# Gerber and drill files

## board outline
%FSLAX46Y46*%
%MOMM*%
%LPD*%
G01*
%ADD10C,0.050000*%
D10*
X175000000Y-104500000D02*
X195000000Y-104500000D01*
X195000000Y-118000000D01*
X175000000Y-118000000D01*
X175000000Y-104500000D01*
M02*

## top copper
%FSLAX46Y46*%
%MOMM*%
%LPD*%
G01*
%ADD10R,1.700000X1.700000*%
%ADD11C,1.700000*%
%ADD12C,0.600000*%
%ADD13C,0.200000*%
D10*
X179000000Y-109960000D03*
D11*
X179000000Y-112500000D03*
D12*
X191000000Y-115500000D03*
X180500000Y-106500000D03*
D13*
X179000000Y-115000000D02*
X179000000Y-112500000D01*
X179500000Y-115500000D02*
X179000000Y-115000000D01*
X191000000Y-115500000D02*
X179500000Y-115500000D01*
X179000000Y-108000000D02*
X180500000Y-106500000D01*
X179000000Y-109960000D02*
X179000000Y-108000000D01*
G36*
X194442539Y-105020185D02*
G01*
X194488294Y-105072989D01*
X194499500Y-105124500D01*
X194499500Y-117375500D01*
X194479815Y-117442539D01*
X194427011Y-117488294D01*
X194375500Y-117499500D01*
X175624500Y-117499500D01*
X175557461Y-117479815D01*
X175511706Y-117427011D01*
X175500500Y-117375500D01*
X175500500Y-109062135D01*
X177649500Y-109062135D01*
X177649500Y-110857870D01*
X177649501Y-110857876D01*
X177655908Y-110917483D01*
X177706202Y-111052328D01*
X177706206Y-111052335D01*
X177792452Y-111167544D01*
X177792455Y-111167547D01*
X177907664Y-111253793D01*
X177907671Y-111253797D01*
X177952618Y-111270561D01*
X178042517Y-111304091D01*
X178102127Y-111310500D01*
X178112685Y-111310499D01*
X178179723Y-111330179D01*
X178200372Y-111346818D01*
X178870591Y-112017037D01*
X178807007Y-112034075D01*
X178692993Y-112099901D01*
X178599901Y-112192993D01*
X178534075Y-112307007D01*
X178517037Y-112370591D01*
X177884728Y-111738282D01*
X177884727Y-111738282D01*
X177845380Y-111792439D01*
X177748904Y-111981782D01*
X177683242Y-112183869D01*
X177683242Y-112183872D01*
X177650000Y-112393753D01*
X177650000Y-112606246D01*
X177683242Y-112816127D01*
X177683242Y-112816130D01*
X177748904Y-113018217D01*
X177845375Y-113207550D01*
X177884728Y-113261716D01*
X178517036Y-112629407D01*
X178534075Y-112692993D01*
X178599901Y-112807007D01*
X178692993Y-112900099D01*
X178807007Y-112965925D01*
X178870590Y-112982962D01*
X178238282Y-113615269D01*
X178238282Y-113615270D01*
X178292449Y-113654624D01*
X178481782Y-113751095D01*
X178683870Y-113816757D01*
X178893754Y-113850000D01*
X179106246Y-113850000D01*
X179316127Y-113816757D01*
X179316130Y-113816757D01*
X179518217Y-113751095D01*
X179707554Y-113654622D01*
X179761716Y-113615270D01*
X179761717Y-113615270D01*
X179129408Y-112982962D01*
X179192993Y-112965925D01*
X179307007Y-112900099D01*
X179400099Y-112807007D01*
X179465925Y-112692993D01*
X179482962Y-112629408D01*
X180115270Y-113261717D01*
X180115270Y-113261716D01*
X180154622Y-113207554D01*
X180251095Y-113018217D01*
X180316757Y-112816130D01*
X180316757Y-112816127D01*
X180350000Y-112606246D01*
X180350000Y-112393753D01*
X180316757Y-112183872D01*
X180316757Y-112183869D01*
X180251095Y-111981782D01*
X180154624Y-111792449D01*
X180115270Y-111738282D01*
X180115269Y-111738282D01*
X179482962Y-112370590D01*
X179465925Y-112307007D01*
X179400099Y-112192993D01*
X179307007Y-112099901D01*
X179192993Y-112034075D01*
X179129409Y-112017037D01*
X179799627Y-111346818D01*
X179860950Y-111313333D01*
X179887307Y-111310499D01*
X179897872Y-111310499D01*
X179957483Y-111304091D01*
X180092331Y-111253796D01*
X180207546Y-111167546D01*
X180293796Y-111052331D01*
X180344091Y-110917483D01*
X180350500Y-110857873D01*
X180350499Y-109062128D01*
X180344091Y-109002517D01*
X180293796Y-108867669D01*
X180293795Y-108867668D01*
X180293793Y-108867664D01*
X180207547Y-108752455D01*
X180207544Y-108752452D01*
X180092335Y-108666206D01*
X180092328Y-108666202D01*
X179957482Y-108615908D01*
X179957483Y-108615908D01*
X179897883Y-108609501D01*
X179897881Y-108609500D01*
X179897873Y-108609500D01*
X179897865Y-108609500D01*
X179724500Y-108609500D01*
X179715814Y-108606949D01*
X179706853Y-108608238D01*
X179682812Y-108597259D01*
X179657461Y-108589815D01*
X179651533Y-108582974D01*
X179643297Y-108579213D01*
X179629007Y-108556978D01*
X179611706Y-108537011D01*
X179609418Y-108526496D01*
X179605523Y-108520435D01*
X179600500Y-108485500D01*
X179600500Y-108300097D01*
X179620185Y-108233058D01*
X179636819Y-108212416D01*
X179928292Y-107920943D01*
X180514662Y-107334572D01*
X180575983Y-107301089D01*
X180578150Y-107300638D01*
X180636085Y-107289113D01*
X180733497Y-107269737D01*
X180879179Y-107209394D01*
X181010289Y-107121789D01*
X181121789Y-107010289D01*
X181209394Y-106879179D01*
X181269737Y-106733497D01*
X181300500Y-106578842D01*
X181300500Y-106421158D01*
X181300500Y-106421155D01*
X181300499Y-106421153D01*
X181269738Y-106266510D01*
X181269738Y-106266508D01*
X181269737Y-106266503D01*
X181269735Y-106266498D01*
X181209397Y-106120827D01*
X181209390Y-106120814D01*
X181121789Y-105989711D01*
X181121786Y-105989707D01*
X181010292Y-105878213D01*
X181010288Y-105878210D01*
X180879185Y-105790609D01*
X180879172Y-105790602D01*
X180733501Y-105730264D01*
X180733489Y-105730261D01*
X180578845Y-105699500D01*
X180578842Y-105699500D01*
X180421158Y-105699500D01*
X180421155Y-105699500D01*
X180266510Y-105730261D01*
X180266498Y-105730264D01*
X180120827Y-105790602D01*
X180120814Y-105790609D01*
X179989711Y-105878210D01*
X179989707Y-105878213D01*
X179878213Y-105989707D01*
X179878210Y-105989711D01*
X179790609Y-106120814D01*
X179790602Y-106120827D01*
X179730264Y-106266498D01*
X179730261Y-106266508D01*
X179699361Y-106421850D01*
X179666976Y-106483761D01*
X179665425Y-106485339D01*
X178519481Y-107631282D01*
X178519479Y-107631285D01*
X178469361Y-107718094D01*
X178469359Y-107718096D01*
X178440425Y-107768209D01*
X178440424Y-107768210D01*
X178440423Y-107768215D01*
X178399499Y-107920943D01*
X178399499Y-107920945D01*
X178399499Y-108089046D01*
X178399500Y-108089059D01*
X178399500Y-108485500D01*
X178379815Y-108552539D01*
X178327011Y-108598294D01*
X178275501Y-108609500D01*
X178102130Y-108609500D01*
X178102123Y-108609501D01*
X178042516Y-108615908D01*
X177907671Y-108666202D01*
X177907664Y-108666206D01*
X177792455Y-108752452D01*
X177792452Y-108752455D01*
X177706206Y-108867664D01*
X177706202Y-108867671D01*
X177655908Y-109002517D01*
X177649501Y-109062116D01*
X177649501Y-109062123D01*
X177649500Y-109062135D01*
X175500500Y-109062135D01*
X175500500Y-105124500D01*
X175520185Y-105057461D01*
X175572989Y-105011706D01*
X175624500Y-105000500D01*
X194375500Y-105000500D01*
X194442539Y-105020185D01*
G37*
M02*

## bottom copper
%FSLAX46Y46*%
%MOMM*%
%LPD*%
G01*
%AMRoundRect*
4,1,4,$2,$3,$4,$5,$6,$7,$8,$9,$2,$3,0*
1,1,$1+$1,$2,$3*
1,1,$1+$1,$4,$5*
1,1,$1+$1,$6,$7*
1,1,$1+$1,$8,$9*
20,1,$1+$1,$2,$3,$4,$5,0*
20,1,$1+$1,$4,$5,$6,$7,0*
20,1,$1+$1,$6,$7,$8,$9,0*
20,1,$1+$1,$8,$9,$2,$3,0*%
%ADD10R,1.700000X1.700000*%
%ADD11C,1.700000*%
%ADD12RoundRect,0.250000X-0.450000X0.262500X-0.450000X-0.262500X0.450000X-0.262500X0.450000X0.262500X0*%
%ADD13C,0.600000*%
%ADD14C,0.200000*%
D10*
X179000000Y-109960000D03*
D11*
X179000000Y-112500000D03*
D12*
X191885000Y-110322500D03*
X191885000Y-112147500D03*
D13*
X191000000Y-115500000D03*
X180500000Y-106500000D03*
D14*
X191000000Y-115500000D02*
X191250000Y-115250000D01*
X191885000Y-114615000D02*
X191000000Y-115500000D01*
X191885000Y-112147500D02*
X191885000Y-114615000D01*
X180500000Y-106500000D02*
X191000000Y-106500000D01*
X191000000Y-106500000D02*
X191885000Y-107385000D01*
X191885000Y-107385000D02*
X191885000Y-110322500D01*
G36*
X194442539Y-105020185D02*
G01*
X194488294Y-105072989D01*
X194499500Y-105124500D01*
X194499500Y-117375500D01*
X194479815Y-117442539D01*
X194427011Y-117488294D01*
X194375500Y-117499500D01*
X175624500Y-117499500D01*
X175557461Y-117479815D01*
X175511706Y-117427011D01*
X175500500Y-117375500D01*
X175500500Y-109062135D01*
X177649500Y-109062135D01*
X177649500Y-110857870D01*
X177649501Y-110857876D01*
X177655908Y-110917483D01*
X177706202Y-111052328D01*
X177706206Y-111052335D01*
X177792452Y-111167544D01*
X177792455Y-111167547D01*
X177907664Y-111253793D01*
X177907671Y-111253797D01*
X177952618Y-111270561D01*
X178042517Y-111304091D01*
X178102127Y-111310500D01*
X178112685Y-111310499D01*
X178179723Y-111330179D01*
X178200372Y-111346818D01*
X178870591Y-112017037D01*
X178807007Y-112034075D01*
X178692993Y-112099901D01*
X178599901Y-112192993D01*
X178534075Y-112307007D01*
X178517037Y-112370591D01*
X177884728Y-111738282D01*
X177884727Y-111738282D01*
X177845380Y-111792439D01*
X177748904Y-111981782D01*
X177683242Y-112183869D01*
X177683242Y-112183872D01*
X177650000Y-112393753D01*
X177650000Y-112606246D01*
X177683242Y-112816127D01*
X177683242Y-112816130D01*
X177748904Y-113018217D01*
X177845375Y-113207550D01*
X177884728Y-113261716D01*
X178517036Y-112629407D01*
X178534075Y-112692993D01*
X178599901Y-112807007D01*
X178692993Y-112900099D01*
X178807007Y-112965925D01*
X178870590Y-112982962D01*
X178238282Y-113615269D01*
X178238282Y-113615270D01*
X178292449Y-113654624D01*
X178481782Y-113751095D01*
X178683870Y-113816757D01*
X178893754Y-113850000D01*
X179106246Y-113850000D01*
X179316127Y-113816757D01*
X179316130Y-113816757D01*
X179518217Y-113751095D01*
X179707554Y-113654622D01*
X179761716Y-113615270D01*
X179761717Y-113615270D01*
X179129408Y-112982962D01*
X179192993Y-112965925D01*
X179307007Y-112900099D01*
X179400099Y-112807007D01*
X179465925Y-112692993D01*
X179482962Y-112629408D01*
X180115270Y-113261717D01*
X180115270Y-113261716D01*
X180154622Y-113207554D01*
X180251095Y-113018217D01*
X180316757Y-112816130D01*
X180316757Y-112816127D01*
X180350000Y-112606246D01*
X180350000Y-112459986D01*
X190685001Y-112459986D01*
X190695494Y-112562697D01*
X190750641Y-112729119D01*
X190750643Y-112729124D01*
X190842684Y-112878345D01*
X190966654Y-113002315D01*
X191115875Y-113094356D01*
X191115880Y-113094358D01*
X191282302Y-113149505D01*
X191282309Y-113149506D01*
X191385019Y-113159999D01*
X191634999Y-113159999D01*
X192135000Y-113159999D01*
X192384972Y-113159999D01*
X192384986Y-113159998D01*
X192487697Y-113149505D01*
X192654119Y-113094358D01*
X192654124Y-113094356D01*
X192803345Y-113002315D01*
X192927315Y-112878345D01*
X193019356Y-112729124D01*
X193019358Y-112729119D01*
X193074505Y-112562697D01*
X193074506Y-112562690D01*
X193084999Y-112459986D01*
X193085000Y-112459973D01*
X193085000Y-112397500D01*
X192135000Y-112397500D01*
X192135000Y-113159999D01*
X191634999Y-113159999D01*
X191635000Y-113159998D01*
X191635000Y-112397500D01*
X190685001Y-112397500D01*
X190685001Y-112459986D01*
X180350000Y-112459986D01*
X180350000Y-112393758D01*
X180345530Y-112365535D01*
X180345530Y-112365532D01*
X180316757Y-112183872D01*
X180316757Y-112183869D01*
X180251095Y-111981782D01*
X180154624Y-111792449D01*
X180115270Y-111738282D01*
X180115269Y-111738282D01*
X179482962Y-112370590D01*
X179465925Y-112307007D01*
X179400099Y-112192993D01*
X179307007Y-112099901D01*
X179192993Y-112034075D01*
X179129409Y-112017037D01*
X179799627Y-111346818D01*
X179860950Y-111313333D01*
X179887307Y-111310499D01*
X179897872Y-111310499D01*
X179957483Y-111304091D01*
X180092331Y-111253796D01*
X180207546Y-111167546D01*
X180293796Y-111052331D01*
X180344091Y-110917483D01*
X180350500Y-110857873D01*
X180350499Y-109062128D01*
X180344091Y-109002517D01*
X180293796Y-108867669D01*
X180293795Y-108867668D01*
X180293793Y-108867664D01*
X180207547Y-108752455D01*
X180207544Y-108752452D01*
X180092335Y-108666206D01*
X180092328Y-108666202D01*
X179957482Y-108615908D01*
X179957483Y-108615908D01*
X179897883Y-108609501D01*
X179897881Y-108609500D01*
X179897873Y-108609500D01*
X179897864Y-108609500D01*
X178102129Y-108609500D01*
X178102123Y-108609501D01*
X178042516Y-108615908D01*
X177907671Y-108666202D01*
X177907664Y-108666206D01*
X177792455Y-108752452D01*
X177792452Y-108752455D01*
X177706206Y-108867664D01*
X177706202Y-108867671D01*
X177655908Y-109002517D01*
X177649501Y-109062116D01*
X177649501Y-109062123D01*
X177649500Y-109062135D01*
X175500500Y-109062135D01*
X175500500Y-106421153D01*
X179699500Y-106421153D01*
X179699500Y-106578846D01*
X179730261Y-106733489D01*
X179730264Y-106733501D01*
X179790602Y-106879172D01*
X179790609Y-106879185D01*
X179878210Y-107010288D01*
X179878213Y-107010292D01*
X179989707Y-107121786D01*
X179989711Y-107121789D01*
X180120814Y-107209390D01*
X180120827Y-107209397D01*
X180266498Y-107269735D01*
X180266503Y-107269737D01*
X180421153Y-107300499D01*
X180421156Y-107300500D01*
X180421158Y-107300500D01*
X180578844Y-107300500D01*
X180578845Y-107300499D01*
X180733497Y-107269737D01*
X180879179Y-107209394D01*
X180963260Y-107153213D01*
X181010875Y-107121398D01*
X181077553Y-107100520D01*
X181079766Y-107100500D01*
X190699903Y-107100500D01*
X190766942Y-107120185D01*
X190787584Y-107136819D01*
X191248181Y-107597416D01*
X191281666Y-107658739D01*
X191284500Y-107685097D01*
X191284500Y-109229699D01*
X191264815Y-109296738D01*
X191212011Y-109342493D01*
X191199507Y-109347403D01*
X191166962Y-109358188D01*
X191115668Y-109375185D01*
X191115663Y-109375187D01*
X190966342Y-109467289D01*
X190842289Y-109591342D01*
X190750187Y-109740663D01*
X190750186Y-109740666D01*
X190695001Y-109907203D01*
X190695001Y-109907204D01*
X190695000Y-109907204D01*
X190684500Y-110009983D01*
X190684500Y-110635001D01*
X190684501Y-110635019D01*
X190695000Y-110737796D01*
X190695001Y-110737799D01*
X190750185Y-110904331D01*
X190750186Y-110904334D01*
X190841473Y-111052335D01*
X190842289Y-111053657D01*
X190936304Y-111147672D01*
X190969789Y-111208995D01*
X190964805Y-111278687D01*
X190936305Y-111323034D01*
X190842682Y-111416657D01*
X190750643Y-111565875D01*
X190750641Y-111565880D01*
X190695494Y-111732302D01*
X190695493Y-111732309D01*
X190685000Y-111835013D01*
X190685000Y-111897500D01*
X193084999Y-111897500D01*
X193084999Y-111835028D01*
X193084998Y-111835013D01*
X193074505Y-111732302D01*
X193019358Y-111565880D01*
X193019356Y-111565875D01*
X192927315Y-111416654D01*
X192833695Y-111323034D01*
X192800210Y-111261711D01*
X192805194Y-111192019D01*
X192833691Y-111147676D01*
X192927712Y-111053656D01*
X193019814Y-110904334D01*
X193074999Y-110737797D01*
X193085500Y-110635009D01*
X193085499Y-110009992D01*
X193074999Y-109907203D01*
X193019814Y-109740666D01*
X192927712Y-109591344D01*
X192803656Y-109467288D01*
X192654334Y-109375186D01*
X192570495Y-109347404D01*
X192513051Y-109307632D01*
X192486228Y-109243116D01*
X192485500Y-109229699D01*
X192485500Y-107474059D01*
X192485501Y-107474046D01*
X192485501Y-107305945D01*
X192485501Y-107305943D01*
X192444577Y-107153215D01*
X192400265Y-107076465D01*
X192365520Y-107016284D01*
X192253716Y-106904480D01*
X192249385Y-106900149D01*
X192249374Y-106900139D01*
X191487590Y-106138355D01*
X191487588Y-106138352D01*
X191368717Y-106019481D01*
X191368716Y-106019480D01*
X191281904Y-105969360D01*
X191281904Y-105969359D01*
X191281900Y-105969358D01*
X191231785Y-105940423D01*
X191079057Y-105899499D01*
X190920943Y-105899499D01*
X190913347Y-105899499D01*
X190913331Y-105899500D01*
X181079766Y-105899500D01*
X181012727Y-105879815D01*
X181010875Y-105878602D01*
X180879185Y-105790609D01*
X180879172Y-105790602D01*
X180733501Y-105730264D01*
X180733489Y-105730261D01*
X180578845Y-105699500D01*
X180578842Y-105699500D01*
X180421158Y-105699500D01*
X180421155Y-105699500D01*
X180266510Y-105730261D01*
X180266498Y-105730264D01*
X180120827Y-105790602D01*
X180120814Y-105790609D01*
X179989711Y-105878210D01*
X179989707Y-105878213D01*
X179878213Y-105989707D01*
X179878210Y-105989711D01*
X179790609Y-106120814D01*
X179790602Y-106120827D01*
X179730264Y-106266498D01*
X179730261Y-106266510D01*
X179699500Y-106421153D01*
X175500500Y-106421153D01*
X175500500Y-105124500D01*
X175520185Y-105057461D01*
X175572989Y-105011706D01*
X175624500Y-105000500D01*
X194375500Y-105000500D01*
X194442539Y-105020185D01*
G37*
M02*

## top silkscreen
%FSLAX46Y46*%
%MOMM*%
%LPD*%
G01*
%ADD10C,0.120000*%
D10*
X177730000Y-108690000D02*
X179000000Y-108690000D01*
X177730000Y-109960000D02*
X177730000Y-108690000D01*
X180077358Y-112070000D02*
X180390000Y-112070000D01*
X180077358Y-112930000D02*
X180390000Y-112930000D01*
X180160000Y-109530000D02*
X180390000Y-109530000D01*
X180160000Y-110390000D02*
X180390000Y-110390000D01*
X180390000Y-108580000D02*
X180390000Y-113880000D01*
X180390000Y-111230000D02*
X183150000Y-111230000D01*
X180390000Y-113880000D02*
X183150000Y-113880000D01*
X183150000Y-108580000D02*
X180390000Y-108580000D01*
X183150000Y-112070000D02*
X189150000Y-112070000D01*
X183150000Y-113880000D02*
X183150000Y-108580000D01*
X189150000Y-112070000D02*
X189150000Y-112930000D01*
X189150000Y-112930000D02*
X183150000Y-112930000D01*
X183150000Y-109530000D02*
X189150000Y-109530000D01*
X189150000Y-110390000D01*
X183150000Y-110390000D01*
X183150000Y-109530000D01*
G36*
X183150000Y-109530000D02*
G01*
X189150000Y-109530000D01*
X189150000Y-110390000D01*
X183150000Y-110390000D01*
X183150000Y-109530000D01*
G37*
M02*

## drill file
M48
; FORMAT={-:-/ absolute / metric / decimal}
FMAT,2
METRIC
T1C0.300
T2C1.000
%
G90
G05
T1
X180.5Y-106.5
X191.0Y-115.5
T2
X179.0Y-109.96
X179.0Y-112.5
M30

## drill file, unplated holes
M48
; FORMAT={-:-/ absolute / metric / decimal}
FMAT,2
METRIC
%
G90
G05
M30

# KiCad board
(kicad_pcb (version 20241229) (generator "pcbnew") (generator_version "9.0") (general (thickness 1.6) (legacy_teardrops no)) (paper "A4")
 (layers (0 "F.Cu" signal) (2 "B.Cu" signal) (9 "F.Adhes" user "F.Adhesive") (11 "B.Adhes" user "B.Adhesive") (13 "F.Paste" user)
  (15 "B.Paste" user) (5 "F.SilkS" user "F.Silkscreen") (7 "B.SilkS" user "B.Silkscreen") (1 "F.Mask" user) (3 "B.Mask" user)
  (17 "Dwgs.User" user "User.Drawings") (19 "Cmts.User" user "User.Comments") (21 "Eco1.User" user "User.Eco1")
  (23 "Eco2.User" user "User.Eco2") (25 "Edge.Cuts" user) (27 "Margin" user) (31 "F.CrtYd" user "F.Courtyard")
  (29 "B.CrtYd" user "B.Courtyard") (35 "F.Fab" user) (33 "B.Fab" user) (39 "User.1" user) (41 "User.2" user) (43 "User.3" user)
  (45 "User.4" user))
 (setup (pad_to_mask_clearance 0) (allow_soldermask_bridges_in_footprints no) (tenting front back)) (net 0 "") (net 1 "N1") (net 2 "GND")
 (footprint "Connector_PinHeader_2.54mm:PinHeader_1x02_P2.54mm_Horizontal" (layer "F.Cu") (at 179 109.96)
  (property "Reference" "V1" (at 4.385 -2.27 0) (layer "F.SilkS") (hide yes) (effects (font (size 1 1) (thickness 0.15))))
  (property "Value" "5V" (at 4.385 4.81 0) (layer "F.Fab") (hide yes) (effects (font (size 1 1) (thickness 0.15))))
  (fp_line (start -1.27 -1.27) (end 0 -1.27) (stroke (width 0.12) (type solid)) (layer "F.SilkS"))
  (fp_line (start -1.27 0) (end -1.27 -1.27) (stroke (width 0.12) (type solid)) (layer "F.SilkS"))
  (fp_line (start 1.077358 2.11) (end 1.39 2.11) (stroke (width 0.12) (type solid)) (layer "F.SilkS"))
  (fp_line (start 1.077358 2.97) (end 1.39 2.97) (stroke (width 0.12) (type solid)) (layer "F.SilkS"))
  (fp_line (start 1.16 -0.43) (end 1.39 -0.43) (stroke (width 0.12) (type solid)) (layer "F.SilkS"))
  (fp_line (start 1.16 0.43) (end 1.39 0.43) (stroke (width 0.12) (type solid)) (layer "F.SilkS"))
  (fp_line (start 1.39 -1.38) (end 1.39 3.92) (stroke (width 0.12) (type solid)) (layer "F.SilkS"))
  (fp_line (start 1.39 1.27) (end 4.15 1.27) (stroke (width 0.12) (type solid)) (layer "F.SilkS"))
  (fp_line (start 1.39 3.92) (end 4.15 3.92) (stroke (width 0.12) (type solid)) (layer "F.SilkS"))
  (fp_line (start 4.15 -1.38) (end 1.39 -1.38) (stroke (width 0.12) (type solid)) (layer "F.SilkS"))
  (fp_line (start 4.15 2.11) (end 10.15 2.11) (stroke (width 0.12) (type solid)) (layer "F.SilkS"))
  (fp_line (start 4.15 3.92) (end 4.15 -1.38) (stroke (width 0.12) (type solid)) (layer "F.SilkS"))
  (fp_line (start 10.15 2.11) (end 10.15 2.97) (stroke (width 0.12) (type solid)) (layer "F.SilkS"))
  (fp_line (start 10.15 2.97) (end 4.15 2.97) (stroke (width 0.12) (type solid)) (layer "F.SilkS"))
  (fp_rect (start 4.15 -0.43) (end 10.15 0.43) (stroke (width 0.12) (type solid)) (fill yes) (layer "F.SilkS"))
  (pad "1" thru_hole rect (at 0 0) (size 1.7 1.7) (drill 1) (layers "*.Cu" "*.Mask") (remove_unused_layers no) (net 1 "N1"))
  (pad "2" thru_hole circle (at 0 2.54) (size 1.7 1.7) (drill 1) (layers "*.Cu" "*.Mask") (remove_unused_layers no) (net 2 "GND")))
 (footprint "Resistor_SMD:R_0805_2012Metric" (layer "B.Cu") (at 191.885 111.235 -90)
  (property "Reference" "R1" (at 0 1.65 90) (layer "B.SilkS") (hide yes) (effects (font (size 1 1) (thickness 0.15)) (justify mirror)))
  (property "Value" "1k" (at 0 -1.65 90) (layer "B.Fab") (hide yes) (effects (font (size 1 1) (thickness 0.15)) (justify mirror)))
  (pad "1" smd roundrect (at -0.9125 0 270) (size 1.025 1.4) (layers "B.Cu" "B.Mask" "B.Paste") (roundrect_rratio 0.243902) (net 1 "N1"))
  (pad "2" smd roundrect (at 0.9125 0 270) (size 1.025 1.4) (layers "B.Cu" "B.Mask" "B.Paste") (roundrect_rratio 0.243902) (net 2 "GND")))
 (gr_rect (start 175 104.5) (end 195 118) (stroke (width 0.05) (type default)) (fill no) (layer "Edge.Cuts"))
 (segment (start 179 109.96) (end 179 108) (width 0.2) (layer "F.Cu") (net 1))
 (segment (start 179 108) (end 180.5 106.5) (width 0.2) (layer "F.Cu") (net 1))
 (via (at 180.5 106.5) (size 0.6) (drill 0.3) (layers "F.Cu" "B.Cu") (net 1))
 (segment (start 191 106.5) (end 191.885 107.385) (width 0.2) (layer "B.Cu") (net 1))
 (segment (start 191.885 107.385) (end 191.885 110.3225) (width 0.2) (layer "B.Cu") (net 1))
 (segment (start 180.5 106.5) (end 191 106.5) (width 0.2) (layer "B.Cu") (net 1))
 (segment (start 179.5 115.5) (end 179 115) (width 0.2) (layer "F.Cu") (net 2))
 (segment (start 179 115) (end 179 112.5) (width 0.2) (layer "F.Cu") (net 2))
 (segment (start 191 115.5) (end 179.5 115.5) (width 0.2) (layer "F.Cu") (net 2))
 (via (at 191 115.5) (size 0.6) (drill 0.3) (layers "F.Cu" "B.Cu") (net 2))
 (segment (start 191.885 112.1475) (end 191.885 114.615) (width 0.2) (layer "B.Cu") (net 2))
 (segment (start 191.885 114.615) (end 191 115.5) (width 0.2) (layer "B.Cu") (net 2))
 (segment (start 191 115.5) (end 191.25 115.25) (width 0.2) (layer "B.Cu") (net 2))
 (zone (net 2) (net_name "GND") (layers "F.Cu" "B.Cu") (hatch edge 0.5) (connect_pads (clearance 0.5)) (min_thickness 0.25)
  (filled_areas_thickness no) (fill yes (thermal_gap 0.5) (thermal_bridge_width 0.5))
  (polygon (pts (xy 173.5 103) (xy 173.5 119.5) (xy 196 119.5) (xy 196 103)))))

